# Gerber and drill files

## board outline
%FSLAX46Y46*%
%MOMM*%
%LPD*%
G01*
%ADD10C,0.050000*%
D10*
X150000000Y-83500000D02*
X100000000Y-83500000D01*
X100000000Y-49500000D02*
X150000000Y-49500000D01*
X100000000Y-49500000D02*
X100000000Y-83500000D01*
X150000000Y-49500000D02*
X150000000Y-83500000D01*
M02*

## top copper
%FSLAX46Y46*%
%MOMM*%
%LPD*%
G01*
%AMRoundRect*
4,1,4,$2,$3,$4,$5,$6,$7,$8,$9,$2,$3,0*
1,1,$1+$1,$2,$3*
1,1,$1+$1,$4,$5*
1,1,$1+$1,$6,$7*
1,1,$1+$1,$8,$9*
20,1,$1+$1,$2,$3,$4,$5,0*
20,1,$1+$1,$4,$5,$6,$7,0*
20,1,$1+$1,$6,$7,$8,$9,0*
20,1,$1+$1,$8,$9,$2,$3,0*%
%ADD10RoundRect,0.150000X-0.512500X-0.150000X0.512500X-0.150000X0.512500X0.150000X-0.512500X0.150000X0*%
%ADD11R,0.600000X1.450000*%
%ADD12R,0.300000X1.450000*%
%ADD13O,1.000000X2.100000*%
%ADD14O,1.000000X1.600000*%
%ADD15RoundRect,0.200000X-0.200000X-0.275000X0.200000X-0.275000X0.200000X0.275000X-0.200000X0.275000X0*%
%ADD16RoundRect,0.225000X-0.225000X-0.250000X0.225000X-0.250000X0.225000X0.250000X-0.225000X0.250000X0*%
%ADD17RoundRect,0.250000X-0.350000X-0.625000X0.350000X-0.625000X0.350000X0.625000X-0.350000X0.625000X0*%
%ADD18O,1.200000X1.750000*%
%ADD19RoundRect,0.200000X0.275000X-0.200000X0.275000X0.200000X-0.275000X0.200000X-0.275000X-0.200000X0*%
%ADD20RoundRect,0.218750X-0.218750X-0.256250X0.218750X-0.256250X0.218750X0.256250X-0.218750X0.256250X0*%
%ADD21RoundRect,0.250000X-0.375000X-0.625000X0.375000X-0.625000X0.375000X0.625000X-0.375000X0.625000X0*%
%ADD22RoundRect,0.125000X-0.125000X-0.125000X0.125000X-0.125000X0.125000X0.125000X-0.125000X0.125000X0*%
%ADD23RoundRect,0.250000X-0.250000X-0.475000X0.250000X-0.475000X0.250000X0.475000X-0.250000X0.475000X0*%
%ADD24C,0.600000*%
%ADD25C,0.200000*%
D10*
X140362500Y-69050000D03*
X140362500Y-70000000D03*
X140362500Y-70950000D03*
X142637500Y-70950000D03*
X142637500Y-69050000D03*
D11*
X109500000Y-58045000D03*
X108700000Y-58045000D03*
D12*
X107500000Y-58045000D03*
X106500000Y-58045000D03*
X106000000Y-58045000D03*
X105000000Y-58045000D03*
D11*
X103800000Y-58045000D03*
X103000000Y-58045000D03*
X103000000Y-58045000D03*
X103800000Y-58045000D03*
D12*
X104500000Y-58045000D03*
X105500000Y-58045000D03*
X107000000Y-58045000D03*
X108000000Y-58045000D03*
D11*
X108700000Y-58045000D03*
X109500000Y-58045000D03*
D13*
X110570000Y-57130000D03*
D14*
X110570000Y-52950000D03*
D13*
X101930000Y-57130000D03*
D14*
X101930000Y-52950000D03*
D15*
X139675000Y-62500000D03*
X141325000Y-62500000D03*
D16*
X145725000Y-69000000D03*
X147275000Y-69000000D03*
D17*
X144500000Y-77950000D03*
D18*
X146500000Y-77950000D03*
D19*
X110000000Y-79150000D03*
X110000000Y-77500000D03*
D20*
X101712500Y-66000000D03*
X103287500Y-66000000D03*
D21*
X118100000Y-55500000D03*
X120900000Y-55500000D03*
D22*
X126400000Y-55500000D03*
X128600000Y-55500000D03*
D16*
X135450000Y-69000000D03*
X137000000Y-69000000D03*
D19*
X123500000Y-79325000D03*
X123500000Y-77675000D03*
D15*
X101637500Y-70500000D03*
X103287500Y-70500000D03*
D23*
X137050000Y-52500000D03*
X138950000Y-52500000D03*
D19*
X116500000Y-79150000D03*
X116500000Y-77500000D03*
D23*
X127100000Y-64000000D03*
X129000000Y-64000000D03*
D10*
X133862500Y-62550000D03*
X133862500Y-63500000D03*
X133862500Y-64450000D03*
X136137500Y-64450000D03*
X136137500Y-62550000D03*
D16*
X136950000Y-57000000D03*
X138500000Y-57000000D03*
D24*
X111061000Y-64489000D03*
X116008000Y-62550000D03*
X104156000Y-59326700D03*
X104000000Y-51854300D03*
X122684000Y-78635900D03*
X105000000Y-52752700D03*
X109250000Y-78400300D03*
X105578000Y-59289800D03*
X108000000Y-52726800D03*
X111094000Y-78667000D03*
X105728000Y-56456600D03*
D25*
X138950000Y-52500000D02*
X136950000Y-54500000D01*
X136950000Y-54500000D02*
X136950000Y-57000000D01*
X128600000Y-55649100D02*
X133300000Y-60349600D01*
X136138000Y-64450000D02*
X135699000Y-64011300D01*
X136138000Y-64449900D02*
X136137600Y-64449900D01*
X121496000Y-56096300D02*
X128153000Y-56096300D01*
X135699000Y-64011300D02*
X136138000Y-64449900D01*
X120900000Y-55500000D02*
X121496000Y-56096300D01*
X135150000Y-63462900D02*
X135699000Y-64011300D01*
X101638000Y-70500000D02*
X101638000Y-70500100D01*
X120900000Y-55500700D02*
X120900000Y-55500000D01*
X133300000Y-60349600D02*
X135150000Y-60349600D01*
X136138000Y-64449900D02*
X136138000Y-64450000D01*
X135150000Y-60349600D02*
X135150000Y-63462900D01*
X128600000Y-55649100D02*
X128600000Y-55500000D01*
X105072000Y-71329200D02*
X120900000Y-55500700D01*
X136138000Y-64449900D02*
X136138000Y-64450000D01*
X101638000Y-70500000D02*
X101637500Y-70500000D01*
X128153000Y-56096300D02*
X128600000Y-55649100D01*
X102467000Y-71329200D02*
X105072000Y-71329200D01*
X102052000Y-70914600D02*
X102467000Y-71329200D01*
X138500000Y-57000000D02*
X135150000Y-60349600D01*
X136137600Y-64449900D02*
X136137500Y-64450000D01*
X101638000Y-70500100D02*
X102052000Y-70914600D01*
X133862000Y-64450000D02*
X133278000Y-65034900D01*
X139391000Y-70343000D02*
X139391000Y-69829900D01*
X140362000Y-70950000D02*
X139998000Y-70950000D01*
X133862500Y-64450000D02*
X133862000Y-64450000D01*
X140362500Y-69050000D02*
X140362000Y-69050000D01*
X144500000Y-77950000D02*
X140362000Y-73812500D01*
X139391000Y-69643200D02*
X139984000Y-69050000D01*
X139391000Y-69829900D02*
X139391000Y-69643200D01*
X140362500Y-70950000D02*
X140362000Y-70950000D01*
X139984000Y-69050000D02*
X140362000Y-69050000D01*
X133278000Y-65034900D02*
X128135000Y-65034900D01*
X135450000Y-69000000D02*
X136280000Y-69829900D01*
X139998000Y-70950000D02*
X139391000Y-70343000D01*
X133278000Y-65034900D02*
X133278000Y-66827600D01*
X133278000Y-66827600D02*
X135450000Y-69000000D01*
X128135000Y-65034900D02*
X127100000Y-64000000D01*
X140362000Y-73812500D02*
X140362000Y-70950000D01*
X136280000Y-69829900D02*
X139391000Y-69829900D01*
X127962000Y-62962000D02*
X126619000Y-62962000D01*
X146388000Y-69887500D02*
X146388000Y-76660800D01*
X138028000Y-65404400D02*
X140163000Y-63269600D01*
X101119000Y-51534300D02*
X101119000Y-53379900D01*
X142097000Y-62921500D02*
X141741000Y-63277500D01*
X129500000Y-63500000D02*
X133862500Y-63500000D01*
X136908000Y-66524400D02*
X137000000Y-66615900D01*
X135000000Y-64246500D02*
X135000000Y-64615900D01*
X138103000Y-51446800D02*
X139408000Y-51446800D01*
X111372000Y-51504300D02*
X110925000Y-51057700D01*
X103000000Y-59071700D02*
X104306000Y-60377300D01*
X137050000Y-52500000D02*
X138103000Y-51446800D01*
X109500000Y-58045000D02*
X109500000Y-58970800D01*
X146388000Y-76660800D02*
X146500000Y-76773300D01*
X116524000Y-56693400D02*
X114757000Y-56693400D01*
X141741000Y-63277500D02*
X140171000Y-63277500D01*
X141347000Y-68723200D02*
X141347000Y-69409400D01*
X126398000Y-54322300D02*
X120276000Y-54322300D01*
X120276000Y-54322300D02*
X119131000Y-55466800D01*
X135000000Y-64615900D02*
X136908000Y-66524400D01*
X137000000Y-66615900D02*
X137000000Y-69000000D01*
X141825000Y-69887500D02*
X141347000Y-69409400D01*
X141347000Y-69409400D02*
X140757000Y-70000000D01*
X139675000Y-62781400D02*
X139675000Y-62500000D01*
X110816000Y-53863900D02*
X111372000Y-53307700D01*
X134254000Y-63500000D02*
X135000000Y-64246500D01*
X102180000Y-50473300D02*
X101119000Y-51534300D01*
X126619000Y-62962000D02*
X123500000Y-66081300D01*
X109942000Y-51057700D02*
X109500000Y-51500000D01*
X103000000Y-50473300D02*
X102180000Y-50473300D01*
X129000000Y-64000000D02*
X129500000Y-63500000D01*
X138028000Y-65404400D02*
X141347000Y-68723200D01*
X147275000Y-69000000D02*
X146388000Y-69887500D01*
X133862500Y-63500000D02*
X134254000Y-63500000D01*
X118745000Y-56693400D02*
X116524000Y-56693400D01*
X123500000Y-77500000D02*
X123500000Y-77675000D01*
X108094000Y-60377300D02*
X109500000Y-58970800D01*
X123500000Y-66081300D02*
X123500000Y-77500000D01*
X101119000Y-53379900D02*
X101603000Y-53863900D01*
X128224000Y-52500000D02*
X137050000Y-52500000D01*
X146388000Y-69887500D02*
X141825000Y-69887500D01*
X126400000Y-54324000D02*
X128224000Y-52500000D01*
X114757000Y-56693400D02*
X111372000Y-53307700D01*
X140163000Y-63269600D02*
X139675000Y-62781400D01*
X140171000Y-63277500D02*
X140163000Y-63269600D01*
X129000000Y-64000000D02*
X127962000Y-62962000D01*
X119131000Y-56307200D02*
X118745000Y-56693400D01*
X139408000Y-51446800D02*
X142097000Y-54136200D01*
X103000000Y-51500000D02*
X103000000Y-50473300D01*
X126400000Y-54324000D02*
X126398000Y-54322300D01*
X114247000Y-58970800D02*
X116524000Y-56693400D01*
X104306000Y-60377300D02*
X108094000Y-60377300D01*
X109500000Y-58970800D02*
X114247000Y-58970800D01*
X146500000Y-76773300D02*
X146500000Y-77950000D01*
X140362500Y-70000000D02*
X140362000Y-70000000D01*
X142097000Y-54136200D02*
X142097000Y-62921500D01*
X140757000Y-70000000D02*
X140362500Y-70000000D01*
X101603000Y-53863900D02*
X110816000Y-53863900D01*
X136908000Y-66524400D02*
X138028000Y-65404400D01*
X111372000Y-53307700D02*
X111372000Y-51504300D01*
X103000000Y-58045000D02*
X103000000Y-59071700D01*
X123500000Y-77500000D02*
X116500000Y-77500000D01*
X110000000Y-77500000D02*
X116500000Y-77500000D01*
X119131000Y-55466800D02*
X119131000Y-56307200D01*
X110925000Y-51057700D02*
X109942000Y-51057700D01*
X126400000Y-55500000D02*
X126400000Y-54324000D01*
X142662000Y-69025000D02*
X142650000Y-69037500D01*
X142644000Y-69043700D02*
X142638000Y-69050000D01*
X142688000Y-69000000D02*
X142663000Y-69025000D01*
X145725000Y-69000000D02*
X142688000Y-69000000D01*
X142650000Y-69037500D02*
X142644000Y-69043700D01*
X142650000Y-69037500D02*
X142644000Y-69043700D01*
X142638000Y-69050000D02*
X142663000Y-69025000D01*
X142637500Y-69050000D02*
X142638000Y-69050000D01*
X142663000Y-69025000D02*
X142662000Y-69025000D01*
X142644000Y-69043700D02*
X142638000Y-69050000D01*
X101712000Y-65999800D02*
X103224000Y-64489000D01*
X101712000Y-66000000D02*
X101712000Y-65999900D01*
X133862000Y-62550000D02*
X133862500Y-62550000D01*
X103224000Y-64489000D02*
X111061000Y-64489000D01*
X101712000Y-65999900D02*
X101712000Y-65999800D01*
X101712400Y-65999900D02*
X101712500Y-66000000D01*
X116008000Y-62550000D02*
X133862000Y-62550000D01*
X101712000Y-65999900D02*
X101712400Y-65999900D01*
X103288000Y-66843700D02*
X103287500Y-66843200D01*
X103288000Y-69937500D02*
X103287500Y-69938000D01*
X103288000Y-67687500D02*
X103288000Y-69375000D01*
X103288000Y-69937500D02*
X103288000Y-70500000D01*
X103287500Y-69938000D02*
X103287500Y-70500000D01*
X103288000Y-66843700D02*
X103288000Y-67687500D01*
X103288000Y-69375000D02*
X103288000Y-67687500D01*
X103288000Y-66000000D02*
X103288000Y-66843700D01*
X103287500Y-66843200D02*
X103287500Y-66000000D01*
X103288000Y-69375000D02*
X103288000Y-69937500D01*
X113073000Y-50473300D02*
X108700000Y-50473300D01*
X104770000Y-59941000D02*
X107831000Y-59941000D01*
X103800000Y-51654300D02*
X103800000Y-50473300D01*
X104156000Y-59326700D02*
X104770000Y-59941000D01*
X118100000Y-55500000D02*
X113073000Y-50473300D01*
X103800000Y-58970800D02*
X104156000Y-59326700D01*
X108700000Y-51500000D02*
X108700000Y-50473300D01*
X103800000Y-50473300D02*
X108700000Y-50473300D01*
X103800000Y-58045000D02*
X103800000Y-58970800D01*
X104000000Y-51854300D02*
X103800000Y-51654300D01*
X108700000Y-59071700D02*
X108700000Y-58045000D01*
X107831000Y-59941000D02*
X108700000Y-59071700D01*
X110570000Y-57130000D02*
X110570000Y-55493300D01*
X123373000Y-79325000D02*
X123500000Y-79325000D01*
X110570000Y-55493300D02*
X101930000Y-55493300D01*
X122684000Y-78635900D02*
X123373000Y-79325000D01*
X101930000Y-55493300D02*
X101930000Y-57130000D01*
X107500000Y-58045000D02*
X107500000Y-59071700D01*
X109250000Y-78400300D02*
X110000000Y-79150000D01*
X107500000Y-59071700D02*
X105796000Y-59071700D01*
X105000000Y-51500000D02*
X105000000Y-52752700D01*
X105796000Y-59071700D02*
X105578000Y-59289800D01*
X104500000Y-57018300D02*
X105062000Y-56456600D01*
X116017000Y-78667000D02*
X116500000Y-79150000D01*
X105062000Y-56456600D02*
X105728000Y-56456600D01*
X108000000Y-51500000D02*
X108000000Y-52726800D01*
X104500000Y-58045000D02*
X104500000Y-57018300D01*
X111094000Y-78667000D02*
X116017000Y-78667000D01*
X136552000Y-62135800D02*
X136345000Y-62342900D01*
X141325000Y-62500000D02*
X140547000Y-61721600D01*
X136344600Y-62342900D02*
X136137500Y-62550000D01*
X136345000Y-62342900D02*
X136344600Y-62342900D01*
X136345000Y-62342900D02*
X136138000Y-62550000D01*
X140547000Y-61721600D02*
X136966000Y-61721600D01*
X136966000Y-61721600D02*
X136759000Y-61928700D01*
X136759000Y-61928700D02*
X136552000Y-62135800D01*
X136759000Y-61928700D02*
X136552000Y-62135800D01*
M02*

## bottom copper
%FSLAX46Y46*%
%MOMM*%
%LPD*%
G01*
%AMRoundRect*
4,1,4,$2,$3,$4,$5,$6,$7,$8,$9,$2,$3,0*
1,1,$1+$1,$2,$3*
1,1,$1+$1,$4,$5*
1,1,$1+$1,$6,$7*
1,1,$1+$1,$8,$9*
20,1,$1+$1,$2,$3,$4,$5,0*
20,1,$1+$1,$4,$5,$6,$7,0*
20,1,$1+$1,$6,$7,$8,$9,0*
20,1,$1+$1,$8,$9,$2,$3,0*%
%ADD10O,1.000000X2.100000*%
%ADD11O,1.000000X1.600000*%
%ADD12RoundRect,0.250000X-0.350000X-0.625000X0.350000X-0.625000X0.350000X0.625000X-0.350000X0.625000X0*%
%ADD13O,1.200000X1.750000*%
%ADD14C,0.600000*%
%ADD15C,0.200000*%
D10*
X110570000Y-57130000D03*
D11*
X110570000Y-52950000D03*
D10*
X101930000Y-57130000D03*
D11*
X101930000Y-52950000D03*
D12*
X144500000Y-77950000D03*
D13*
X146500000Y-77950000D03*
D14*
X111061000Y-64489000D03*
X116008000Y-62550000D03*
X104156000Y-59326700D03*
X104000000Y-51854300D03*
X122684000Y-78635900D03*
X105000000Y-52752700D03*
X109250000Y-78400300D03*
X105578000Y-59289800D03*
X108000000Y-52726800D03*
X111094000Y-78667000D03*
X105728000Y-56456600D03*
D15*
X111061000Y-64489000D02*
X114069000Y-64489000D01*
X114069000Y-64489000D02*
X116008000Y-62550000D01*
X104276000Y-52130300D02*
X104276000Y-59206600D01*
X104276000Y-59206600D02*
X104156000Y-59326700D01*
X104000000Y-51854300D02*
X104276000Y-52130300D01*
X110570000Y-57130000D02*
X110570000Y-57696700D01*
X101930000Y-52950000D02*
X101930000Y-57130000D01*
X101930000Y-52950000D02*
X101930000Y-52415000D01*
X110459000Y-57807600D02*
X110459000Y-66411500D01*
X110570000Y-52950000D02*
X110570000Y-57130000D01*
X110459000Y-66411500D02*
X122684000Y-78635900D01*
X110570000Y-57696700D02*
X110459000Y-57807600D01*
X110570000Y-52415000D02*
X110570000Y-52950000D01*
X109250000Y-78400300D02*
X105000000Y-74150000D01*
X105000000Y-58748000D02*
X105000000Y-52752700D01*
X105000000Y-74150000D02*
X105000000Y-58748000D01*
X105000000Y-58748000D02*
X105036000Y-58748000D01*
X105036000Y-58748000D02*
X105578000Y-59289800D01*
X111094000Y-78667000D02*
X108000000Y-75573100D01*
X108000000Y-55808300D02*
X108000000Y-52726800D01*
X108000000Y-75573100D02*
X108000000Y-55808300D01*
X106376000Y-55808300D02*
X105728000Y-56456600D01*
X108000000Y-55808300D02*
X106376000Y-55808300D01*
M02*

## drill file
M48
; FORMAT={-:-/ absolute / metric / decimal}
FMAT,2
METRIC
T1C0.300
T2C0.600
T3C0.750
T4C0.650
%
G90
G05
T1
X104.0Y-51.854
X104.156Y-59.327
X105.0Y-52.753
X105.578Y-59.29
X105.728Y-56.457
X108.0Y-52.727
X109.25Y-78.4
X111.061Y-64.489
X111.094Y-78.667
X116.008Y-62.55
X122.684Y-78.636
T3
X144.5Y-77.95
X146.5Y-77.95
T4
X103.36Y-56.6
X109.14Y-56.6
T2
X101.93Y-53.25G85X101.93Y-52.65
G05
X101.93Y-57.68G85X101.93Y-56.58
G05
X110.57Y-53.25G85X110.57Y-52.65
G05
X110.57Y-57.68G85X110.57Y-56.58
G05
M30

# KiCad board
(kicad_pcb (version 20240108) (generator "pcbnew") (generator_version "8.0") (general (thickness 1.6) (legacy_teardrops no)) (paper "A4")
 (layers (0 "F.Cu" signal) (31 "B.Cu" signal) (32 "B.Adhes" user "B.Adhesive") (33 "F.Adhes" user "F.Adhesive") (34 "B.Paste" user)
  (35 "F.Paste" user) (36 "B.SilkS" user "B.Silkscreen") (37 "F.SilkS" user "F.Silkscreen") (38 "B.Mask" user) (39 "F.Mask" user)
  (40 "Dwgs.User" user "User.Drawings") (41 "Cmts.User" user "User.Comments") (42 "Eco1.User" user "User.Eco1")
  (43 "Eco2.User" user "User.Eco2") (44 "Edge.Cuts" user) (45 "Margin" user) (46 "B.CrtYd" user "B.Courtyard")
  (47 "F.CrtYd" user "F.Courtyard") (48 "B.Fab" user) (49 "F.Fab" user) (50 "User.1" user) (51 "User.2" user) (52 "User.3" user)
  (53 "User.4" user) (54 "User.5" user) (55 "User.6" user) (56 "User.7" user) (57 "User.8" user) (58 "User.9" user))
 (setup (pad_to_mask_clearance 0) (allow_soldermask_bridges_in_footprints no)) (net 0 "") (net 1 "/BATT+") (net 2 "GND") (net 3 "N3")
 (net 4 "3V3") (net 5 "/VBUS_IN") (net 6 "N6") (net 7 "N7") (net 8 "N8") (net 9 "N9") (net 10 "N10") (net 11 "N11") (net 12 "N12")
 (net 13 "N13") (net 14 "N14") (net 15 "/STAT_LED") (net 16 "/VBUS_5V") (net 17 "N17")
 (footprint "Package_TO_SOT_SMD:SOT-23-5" (layer "F.Cu") (at 141.5 70)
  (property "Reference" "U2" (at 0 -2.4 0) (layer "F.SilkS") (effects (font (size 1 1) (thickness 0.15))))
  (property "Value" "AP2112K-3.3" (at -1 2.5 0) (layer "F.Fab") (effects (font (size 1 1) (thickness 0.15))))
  (pad "1" smd roundrect (at -1.1375 -0.95) (size 1.325 0.6) (layers "F.Cu" "F.Paste" "F.Mask") (roundrect_rratio 0.25) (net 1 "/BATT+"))
  (pad "2" smd roundrect (at -1.1375 0) (size 1.325 0.6) (layers "F.Cu" "F.Paste" "F.Mask") (roundrect_rratio 0.25) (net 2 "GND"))
  (pad "3" smd roundrect (at -1.1375 0.95) (size 1.325 0.6) (layers "F.Cu" "F.Paste" "F.Mask") (roundrect_rratio 0.25) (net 1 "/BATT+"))
  (pad "4" smd roundrect (at 1.1375 0.95) (size 1.325 0.6) (layers "F.Cu" "F.Paste" "F.Mask") (roundrect_rratio 0.25) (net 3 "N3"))
  (pad "5" smd roundrect (at 1.1375 -0.95) (size 1.325 0.6) (layers "F.Cu" "F.Paste" "F.Mask") (roundrect_rratio 0.25) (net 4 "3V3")))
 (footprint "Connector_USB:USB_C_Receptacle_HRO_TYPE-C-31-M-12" (layer "F.Cu") (at 106.25 54 180)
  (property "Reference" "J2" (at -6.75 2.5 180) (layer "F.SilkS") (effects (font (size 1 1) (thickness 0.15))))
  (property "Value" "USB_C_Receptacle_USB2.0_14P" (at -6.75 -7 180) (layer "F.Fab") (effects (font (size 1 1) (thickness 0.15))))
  (pad "" np_thru_hole circle (at -2.89 -2.6 180) (size 0.65 0.65) (drill 0.65) (layers "*.Cu" "*.Mask"))
  (pad "" np_thru_hole circle (at 2.89 -2.6 180) (size 0.65 0.65) (drill 0.65) (layers "*.Cu" "*.Mask"))
  (pad "A1" smd rect (at -3.25 -4.045 180) (size 0.6 1.45) (layers "F.Cu" "F.Paste" "F.Mask") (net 2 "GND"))
  (pad "A4" smd rect (at -2.45 -4.045 180) (size 0.6 1.45) (layers "F.Cu" "F.Paste" "F.Mask") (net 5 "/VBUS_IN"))
  (pad "A5" smd rect (at -1.25 -4.045 180) (size 0.3 1.45) (layers "F.Cu" "F.Paste" "F.Mask") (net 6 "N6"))
  (pad "A6" smd rect (at -0.25 -4.045 180) (size 0.3 1.45) (layers "F.Cu" "F.Paste" "F.Mask") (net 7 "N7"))
  (pad "A7" smd rect (at 0.25 -4.045 180) (size 0.3 1.45) (layers "F.Cu" "F.Paste" "F.Mask") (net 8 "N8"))
  (pad "A8" smd rect (at 1.25 -4.045 180) (size 0.3 1.45) (layers "F.Cu" "F.Paste" "F.Mask"))
  (pad "A9" smd rect (at 2.45 -4.045 180) (size 0.6 1.45) (layers "F.Cu" "F.Paste" "F.Mask") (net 5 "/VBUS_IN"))
  (pad "A12" smd rect (at 3.25 -4.045 180) (size 0.6 1.45) (layers "F.Cu" "F.Paste" "F.Mask") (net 2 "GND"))
  (pad "B1" smd rect (at 3.25 -4.045 180) (size 0.6 1.45) (layers "F.Cu" "F.Paste" "F.Mask") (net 2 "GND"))
  (pad "B4" smd rect (at 2.45 -4.045 180) (size 0.6 1.45) (layers "F.Cu" "F.Paste" "F.Mask") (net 5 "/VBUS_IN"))
  (pad "B5" smd rect (at 1.75 -4.045 180) (size 0.3 1.45) (layers "F.Cu" "F.Paste" "F.Mask") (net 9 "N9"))
  (pad "B6" smd rect (at 0.75 -4.045 180) (size 0.3 1.45) (layers "F.Cu" "F.Paste" "F.Mask") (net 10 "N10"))
  (pad "B7" smd rect (at -0.75 -4.045 180) (size 0.3 1.45) (layers "F.Cu" "F.Paste" "F.Mask") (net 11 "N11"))
  (pad "B8" smd rect (at -1.75 -4.045 180) (size 0.3 1.45) (layers "F.Cu" "F.Paste" "F.Mask"))
  (pad "B9" smd rect (at -2.45 -4.045 180) (size 0.6 1.45) (layers "F.Cu" "F.Paste" "F.Mask") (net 5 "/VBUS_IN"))
  (pad "B12" smd rect (at -3.25 -4.045 180) (size 0.6 1.45) (layers "F.Cu" "F.Paste" "F.Mask") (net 2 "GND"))
  (pad "S1" thru_hole oval (at -4.32 -3.13 180) (size 1 2.1) (drill oval 0.6 1.7) (layers "*.Cu" "*.Mask") (remove_unused_layers no)
   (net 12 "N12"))
  (pad "S1" thru_hole oval (at -4.32 1.05 180) (size 1 1.6) (drill oval 0.6 1.2) (layers "*.Cu" "*.Mask") (remove_unused_layers no)
   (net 12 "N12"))
  (pad "S1" thru_hole oval (at 4.32 -3.13 180) (size 1 2.1) (drill oval 0.6 1.7) (layers "*.Cu" "*.Mask") (remove_unused_layers no)
   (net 12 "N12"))
  (pad "S1" thru_hole oval (at 4.32 1.05 180) (size 1 1.6) (drill oval 0.6 1.2) (layers "*.Cu" "*.Mask") (remove_unused_layers no)
   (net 12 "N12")))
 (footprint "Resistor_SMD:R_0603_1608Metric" (layer "F.Cu") (at 140.5 62.5)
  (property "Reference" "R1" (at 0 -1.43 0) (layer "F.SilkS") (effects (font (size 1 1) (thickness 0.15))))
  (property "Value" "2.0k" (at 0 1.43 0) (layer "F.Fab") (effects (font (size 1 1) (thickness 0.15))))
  (pad "1" smd roundrect (at -0.825 0) (size 0.8 0.95) (layers "F.Cu" "F.Paste" "F.Mask") (roundrect_rratio 0.25) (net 2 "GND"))
  (pad "2" smd roundrect (at 0.825 0) (size 0.8 0.95) (layers "F.Cu" "F.Paste" "F.Mask") (roundrect_rratio 0.25) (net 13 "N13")))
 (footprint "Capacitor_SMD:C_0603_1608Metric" (layer "F.Cu") (at 146.5 69)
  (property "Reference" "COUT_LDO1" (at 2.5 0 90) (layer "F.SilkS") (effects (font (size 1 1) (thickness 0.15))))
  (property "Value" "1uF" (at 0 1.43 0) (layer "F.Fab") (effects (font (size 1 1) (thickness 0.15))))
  (pad "1" smd roundrect (at -0.775 0) (size 0.9 0.95) (layers "F.Cu" "F.Paste" "F.Mask") (roundrect_rratio 0.25) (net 4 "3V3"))
  (pad "2" smd roundrect (at 0.775 0) (size 0.9 0.95) (layers "F.Cu" "F.Paste" "F.Mask") (roundrect_rratio 0.25) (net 2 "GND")))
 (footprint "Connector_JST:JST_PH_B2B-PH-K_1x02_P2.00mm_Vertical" (layer "F.Cu") (at 144.5 77.95)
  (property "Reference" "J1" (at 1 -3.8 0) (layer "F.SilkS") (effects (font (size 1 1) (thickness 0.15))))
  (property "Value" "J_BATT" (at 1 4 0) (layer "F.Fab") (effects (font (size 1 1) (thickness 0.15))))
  (pad "1" thru_hole roundrect (at 0 0) (size 1.2 1.75) (drill 0.75) (layers "*.Cu" "*.Mask") (remove_unused_layers no)
   (roundrect_rratio 0.208333) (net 1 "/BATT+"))
  (pad "2" thru_hole oval (at 2 0) (size 1.2 1.75) (drill 0.75) (layers "*.Cu" "*.Mask") (remove_unused_layers no) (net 2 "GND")))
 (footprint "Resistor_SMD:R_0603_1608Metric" (layer "F.Cu") (at 110 78.325 90)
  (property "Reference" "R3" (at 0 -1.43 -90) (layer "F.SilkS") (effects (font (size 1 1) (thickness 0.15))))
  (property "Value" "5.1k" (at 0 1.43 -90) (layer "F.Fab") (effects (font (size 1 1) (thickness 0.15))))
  (pad "1" smd roundrect (at -0.825 0 90) (size 0.8 0.95) (layers "F.Cu" "F.Paste" "F.Mask") (roundrect_rratio 0.25) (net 6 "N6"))
  (pad "2" smd roundrect (at 0.825 0 90) (size 0.8 0.95) (layers "F.Cu" "F.Paste" "F.Mask") (roundrect_rratio 0.25) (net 2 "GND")))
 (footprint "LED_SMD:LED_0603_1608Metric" (layer "F.Cu") (at 102.5 66)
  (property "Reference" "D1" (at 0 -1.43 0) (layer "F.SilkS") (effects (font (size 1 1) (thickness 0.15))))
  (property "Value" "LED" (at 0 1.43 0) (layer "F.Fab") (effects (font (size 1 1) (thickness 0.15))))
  (pad "1" smd roundrect (at -0.7875 0) (size 0.875 0.95) (layers "F.Cu" "F.Paste" "F.Mask") (roundrect_rratio 0.25) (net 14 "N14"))
  (pad "2" smd roundrect (at 0.7875 0) (size 0.875 0.95) (layers "F.Cu" "F.Paste" "F.Mask") (roundrect_rratio 0.25) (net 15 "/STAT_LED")))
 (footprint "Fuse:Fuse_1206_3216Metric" (layer "F.Cu") (at 119.5 55.5)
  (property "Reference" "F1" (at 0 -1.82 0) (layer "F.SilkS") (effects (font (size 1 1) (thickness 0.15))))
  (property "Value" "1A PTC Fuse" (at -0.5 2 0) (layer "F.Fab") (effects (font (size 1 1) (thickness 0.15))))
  (pad "1" smd roundrect (at -1.4 0) (size 1.25 1.75) (layers "F.Cu" "F.Paste" "F.Mask") (roundrect_rratio 0.2) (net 5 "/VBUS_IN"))
  (pad "2" smd roundrect (at 1.4 0) (size 1.25 1.75) (layers "F.Cu" "F.Paste" "F.Mask") (roundrect_rratio 0.2) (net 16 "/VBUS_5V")))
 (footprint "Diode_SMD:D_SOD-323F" (layer "F.Cu") (at 127.5 55.5)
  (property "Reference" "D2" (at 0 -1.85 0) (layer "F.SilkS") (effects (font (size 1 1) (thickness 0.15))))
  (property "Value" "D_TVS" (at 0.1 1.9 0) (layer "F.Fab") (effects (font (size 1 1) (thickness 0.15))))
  (pad "1" smd roundrect (at -1.1 0) (size 0.5 0.5) (layers "F.Cu" "F.Paste" "F.Mask") (roundrect_rratio 0.25) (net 2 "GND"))
  (pad "2" smd roundrect (at 1.1 0) (size 0.5 0.5) (layers "F.Cu" "F.Paste" "F.Mask") (roundrect_rratio 0.25) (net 16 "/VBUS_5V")))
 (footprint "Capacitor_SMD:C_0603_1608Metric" (layer "F.Cu") (at 136.225 69)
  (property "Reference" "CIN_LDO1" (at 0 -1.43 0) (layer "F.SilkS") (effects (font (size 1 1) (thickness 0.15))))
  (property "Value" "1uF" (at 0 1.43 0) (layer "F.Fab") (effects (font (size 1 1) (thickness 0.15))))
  (pad "1" smd roundrect (at -0.775 0) (size 0.9 0.95) (layers "F.Cu" "F.Paste" "F.Mask") (roundrect_rratio 0.25) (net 1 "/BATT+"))
  (pad "2" smd roundrect (at 0.775 0) (size 0.9 0.95) (layers "F.Cu" "F.Paste" "F.Mask") (roundrect_rratio 0.25) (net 2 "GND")))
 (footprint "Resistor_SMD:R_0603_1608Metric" (layer "F.Cu") (at 123.5 78.5 90)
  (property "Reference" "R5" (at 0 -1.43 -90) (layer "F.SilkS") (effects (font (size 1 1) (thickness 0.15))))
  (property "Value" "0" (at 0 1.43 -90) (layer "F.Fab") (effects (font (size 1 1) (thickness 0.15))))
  (pad "1" smd roundrect (at -0.825 0 90) (size 0.8 0.95) (layers "F.Cu" "F.Paste" "F.Mask") (roundrect_rratio 0.25) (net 12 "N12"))
  (pad "2" smd roundrect (at 0.825 0 90) (size 0.8 0.95) (layers "F.Cu" "F.Paste" "F.Mask") (roundrect_rratio 0.25) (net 2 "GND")))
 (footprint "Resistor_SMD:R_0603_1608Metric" (layer "F.Cu") (at 102.4625 70.5)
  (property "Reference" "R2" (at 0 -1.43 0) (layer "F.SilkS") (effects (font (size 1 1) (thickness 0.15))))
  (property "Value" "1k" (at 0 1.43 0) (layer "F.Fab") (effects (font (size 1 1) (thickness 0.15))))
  (pad "1" smd roundrect (at -0.825 0) (size 0.8 0.95) (layers "F.Cu" "F.Paste" "F.Mask") (roundrect_rratio 0.25) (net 16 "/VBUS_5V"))
  (pad "2" smd roundrect (at 0.825 0) (size 0.8 0.95) (layers "F.Cu" "F.Paste" "F.Mask") (roundrect_rratio 0.25) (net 15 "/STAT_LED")))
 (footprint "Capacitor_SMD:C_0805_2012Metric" (layer "F.Cu") (at 138 52.5)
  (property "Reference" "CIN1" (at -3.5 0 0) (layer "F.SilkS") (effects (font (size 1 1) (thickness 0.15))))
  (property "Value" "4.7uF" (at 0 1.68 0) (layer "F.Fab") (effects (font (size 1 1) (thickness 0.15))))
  (pad "1" smd roundrect (at -0.95 0) (size 1 1.45) (layers "F.Cu" "F.Paste" "F.Mask") (roundrect_rratio 0.25) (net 2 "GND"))
  (pad "2" smd roundrect (at 0.95 0) (size 1 1.45) (layers "F.Cu" "F.Paste" "F.Mask") (roundrect_rratio 0.25) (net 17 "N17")))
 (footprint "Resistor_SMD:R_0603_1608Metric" (layer "F.Cu") (at 116.5 78.325 90)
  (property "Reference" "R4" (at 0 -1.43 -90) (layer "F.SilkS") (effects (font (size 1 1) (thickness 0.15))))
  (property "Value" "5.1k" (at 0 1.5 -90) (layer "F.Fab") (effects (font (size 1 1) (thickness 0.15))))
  (pad "1" smd roundrect (at -0.825 0 90) (size 0.8 0.95) (layers "F.Cu" "F.Paste" "F.Mask") (roundrect_rratio 0.25) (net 9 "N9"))
  (pad "2" smd roundrect (at 0.825 0 90) (size 0.8 0.95) (layers "F.Cu" "F.Paste" "F.Mask") (roundrect_rratio 0.25) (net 2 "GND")))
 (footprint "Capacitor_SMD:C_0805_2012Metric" (layer "F.Cu") (at 128.05 64)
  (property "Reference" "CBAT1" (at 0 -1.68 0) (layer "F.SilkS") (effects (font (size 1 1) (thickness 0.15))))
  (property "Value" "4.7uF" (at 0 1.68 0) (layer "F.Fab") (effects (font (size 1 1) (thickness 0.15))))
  (pad "1" smd roundrect (at -0.95 0) (size 1 1.45) (layers "F.Cu" "F.Paste" "F.Mask") (roundrect_rratio 0.25) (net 1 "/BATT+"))
  (pad "2" smd roundrect (at 0.95 0) (size 1 1.45) (layers "F.Cu" "F.Paste" "F.Mask") (roundrect_rratio 0.25) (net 2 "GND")))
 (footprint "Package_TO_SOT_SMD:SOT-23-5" (layer "F.Cu") (at 135 63.5)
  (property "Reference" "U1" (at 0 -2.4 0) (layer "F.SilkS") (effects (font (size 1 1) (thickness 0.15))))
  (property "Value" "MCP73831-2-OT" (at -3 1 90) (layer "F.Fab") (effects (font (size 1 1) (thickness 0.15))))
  (pad "1" smd roundrect (at -1.1375 -0.95) (size 1.325 0.6) (layers "F.Cu" "F.Paste" "F.Mask") (roundrect_rratio 0.25) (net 14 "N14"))
  (pad "2" smd roundrect (at -1.1375 0) (size 1.325 0.6) (layers "F.Cu" "F.Paste" "F.Mask") (roundrect_rratio 0.25) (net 2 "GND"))
  (pad "3" smd roundrect (at -1.1375 0.95) (size 1.325 0.6) (layers "F.Cu" "F.Paste" "F.Mask") (roundrect_rratio 0.25) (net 1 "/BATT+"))
  (pad "4" smd roundrect (at 1.1375 0.95) (size 1.325 0.6) (layers "F.Cu" "F.Paste" "F.Mask") (roundrect_rratio 0.25) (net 16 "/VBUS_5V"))
  (pad "5" smd roundrect (at 1.1375 -0.95) (size 1.325 0.6) (layers "F.Cu" "F.Paste" "F.Mask") (roundrect_rratio 0.25) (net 13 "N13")))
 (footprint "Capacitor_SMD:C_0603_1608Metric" (layer "F.Cu") (at 137.725 57)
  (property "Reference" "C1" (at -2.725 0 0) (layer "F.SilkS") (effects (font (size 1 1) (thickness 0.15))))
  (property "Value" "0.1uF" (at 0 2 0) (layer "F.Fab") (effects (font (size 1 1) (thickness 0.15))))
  (pad "1" smd roundrect (at -0.775 0) (size 0.9 0.95) (layers "F.Cu" "F.Paste" "F.Mask") (roundrect_rratio 0.25) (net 17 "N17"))
  (pad "2" smd roundrect (at 0.775 0) (size 0.9 0.95) (layers "F.Cu" "F.Paste" "F.Mask") (roundrect_rratio 0.25) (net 16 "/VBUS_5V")))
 (gr_line (start 150 83.5) (end 100 83.5) (stroke (width 0.05) (type default)) (layer "Edge.Cuts"))
 (gr_line (start 100 49.5) (end 150 49.5) (stroke (width 0.05) (type default)) (layer "Edge.Cuts"))
 (gr_line (start 100 49.5) (end 100 83.5) (stroke (width 0.05) (type default)) (layer "Edge.Cuts"))
 (gr_line (start 150 49.5) (end 150 83.5) (stroke (width 0.05) (type default)) (layer "Edge.Cuts"))
 (segment (start 138.95 52.5) (end 136.95 54.5) (width 0.2) (layer "F.Cu") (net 17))
 (segment (start 136.95 54.5) (end 136.95 57) (width 0.2) (layer "F.Cu") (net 17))
 (segment (start 128.6 55.6491) (end 133.3 60.3496) (width 0.2) (layer "F.Cu") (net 16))
 (segment (start 136.138 64.45) (end 135.699 64.0113) (width 0.2) (layer "F.Cu") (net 16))
 (segment (start 136.138 64.4499) (end 136.1376 64.4499) (width 0.2) (layer "F.Cu") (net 16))
 (segment (start 121.496 56.0963) (end 128.153 56.0963) (width 0.2) (layer "F.Cu") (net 16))
 (segment (start 135.699 64.0113) (end 136.138 64.4499) (width 0.2) (layer "F.Cu") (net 16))
 (segment (start 120.9 55.5) (end 121.496 56.0963) (width 0.2) (layer "F.Cu") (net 16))
 (segment (start 135.15 63.4629) (end 135.699 64.0113) (width 0.2) (layer "F.Cu") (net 16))
 (segment (start 101.638 70.5) (end 101.638 70.5001) (width 0.2) (layer "F.Cu") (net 16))
 (segment (start 120.9 55.5007) (end 120.9 55.5) (width 0.2) (layer "F.Cu") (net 16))
 (segment (start 133.3 60.3496) (end 135.15 60.3496) (width 0.2) (layer "F.Cu") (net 16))
 (segment (start 136.138 64.4499) (end 136.138 64.45) (width 0.2) (layer "F.Cu") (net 16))
 (segment (start 135.15 60.3496) (end 135.15 63.4629) (width 0.2) (layer "F.Cu") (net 16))
 (segment (start 128.6 55.6491) (end 128.6 55.5) (width 0.2) (layer "F.Cu") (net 16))
 (segment (start 105.072 71.3292) (end 120.9 55.5007) (width 0.2) (layer "F.Cu") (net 16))
 (segment (start 136.138 64.4499) (end 136.138 64.45) (width 0.2) (layer "F.Cu") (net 16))
 (segment (start 101.638 70.5) (end 101.6375 70.5) (width 0.2) (layer "F.Cu") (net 16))
 (segment (start 128.153 56.0963) (end 128.6 55.6491) (width 0.2) (layer "F.Cu") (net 16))
 (segment (start 102.467 71.3292) (end 105.072 71.3292) (width 0.2) (layer "F.Cu") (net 16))
 (segment (start 102.052 70.9146) (end 102.467 71.3292) (width 0.2) (layer "F.Cu") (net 16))
 (segment (start 138.5 57) (end 135.15 60.3496) (width 0.2) (layer "F.Cu") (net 16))
 (segment (start 136.1376 64.4499) (end 136.1375 64.45) (width 0.2) (layer "F.Cu") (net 16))
 (segment (start 101.638 70.5001) (end 102.052 70.9146) (width 0.2) (layer "F.Cu") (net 16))
 (segment (start 133.862 64.45) (end 133.278 65.0349) (width 0.2) (layer "F.Cu") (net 1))
 (segment (start 139.391 70.343) (end 139.391 69.8299) (width 0.2) (layer "F.Cu") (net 1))
 (segment (start 140.362 70.95) (end 139.998 70.95) (width 0.2) (layer "F.Cu") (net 1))
 (segment (start 133.8625 64.45) (end 133.862 64.45) (width 0.2) (layer "F.Cu") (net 1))
 (segment (start 140.3625 69.05) (end 140.362 69.05) (width 0.2) (layer "F.Cu") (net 1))
 (segment (start 144.5 77.95) (end 140.362 73.8125) (width 0.2) (layer "F.Cu") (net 1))
 (segment (start 139.391 69.6432) (end 139.984 69.05) (width 0.2) (layer "F.Cu") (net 1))
 (segment (start 139.391 69.8299) (end 139.391 69.6432) (width 0.2) (layer "F.Cu") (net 1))
 (segment (start 140.3625 70.95) (end 140.362 70.95) (width 0.2) (layer "F.Cu") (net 1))
 (segment (start 139.984 69.05) (end 140.362 69.05) (width 0.2) (layer "F.Cu") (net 1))
 (segment (start 133.278 65.0349) (end 128.135 65.0349) (width 0.2) (layer "F.Cu") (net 1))
 (segment (start 135.45 69) (end 136.28 69.8299) (width 0.2) (layer "F.Cu") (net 1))
 (segment (start 139.998 70.95) (end 139.391 70.343) (width 0.2) (layer "F.Cu") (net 1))
 (segment (start 133.278 65.0349) (end 133.278 66.8276) (width 0.2) (layer "F.Cu") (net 1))
 (segment (start 133.278 66.8276) (end 135.45 69) (width 0.2) (layer "F.Cu") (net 1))
 (segment (start 128.135 65.0349) (end 127.1 64) (width 0.2) (layer "F.Cu") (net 1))
 (segment (start 140.362 73.8125) (end 140.362 70.95) (width 0.2) (layer "F.Cu") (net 1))
 (segment (start 136.28 69.8299) (end 139.391 69.8299) (width 0.2) (layer "F.Cu") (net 1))
 (segment (start 127.962 62.962) (end 126.619 62.962) (width 0.2) (layer "F.Cu") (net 2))
 (segment (start 146.388 69.8875) (end 146.388 76.6608) (width 0.2) (layer "F.Cu") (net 2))
 (segment (start 138.028 65.4044) (end 140.163 63.2696) (width 0.2) (layer "F.Cu") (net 2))
 (segment (start 101.119 51.5343) (end 101.119 53.3799) (width 0.2) (layer "F.Cu") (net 2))
 (segment (start 142.097 62.9215) (end 141.741 63.2775) (width 0.2) (layer "F.Cu") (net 2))
 (segment (start 129.5 63.5) (end 133.8625 63.5) (width 0.2) (layer "F.Cu") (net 2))
 (segment (start 136.908 66.5244) (end 137 66.6159) (width 0.2) (layer "F.Cu") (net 2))
 (segment (start 135 64.2465) (end 135 64.6159) (width 0.2) (layer "F.Cu") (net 2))
 (segment (start 138.103 51.4468) (end 139.408 51.4468) (width 0.2) (layer "F.Cu") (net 2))
 (segment (start 111.372 51.5043) (end 110.925 51.0577) (width 0.2) (layer "F.Cu") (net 2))
 (segment (start 103 59.0717) (end 104.306 60.3773) (width 0.2) (layer "F.Cu") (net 2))
 (segment (start 137.05 52.5) (end 138.103 51.4468) (width 0.2) (layer "F.Cu") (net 2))
 (segment (start 109.5 58.045) (end 109.5 58.9708) (width 0.2) (layer "F.Cu") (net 2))
 (segment (start 146.388 76.6608) (end 146.5 76.7733) (width 0.2) (layer "F.Cu") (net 2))
 (segment (start 116.524 56.6934) (end 114.757 56.6934) (width 0.2) (layer "F.Cu") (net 2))
 (segment (start 141.741 63.2775) (end 140.171 63.2775) (width 0.2) (layer "F.Cu") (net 2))
 (segment (start 141.347 68.7232) (end 141.347 69.4094) (width 0.2) (layer "F.Cu") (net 2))
 (segment (start 126.398 54.3223) (end 120.276 54.3223) (width 0.2) (layer "F.Cu") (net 2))
 (segment (start 120.276 54.3223) (end 119.131 55.4668) (width 0.2) (layer "F.Cu") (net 2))
 (segment (start 135 64.6159) (end 136.908 66.5244) (width 0.2) (layer "F.Cu") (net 2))
 (segment (start 137 66.6159) (end 137 69) (width 0.2) (layer "F.Cu") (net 2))
 (segment (start 141.825 69.8875) (end 141.347 69.4094) (width 0.2) (layer "F.Cu") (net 2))
 (segment (start 141.347 69.4094) (end 140.757 70) (width 0.2) (layer "F.Cu") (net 2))
 (segment (start 139.675 62.7814) (end 139.675 62.5) (width 0.2) (layer "F.Cu") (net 2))
 (segment (start 110.816 53.8639) (end 111.372 53.3077) (width 0.2) (layer "F.Cu") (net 2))
 (segment (start 134.254 63.5) (end 135 64.2465) (width 0.2) (layer "F.Cu") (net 2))
 (segment (start 102.18 50.4733) (end 101.119 51.5343) (width 0.2) (layer "F.Cu") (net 2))
 (segment (start 126.619 62.962) (end 123.5 66.0813) (width 0.2) (layer "F.Cu") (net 2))
 (segment (start 109.942 51.0577) (end 109.5 51.5) (width 0.2) (layer "F.Cu") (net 2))
 (segment (start 103 50.4733) (end 102.18 50.4733) (width 0.2) (layer "F.Cu") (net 2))
 (segment (start 129 64) (end 129.5 63.5) (width 0.2) (layer "F.Cu") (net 2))
 (segment (start 138.028 65.4044) (end 141.347 68.7232) (width 0.2) (layer "F.Cu") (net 2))
 (segment (start 147.275 69) (end 146.388 69.8875) (width 0.2) (layer "F.Cu") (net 2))
 (segment (start 133.8625 63.5) (end 134.254 63.5) (width 0.2) (layer "F.Cu") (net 2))
 (segment (start 118.745 56.6934) (end 116.524 56.6934) (width 0.2) (layer "F.Cu") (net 2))
 (segment (start 123.5 77.5) (end 123.5 77.675) (width 0.2) (layer "F.Cu") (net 2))
 (segment (start 108.094 60.3773) (end 109.5 58.9708) (width 0.2) (layer "F.Cu") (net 2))
 (segment (start 123.5 66.0813) (end 123.5 77.5) (width 0.2) (layer "F.Cu") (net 2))
 (segment (start 101.119 53.3799) (end 101.603 53.8639) (width 0.2) (layer "F.Cu") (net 2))
 (segment (start 128.224 52.5) (end 137.05 52.5) (width 0.2) (layer "F.Cu") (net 2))
 (segment (start 146.388 69.8875) (end 141.825 69.8875) (width 0.2) (layer "F.Cu") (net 2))
 (segment (start 126.4 54.324) (end 128.224 52.5) (width 0.2) (layer "F.Cu") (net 2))
 (segment (start 114.757 56.6934) (end 111.372 53.3077) (width 0.2) (layer "F.Cu") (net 2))
 (segment (start 140.163 63.2696) (end 139.675 62.7814) (width 0.2) (layer "F.Cu") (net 2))
 (segment (start 140.171 63.2775) (end 140.163 63.2696) (width 0.2) (layer "F.Cu") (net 2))
 (segment (start 129 64) (end 127.962 62.962) (width 0.2) (layer "F.Cu") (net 2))
 (segment (start 119.131 56.3072) (end 118.745 56.6934) (width 0.2) (layer "F.Cu") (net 2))
 (segment (start 139.408 51.4468) (end 142.097 54.1362) (width 0.2) (layer "F.Cu") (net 2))
 (segment (start 103 51.5) (end 103 50.4733) (width 0.2) (layer "F.Cu") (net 2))
 (segment (start 126.4 54.324) (end 126.398 54.3223) (width 0.2) (layer "F.Cu") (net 2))
 (segment (start 114.247 58.9708) (end 116.524 56.6934) (width 0.2) (layer "F.Cu") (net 2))
 (segment (start 104.306 60.3773) (end 108.094 60.3773) (width 0.2) (layer "F.Cu") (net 2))
 (segment (start 109.5 58.9708) (end 114.247 58.9708) (width 0.2) (layer "F.Cu") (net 2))
 (segment (start 146.5 76.7733) (end 146.5 77.95) (width 0.2) (layer "F.Cu") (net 2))
 (segment (start 140.3625 70) (end 140.362 70) (width 0.2) (layer "F.Cu") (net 2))
 (segment (start 142.097 54.1362) (end 142.097 62.9215) (width 0.2) (layer "F.Cu") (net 2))
 (segment (start 140.757 70) (end 140.3625 70) (width 0.2) (layer "F.Cu") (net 2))
 (segment (start 101.603 53.8639) (end 110.816 53.8639) (width 0.2) (layer "F.Cu") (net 2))
 (segment (start 136.908 66.5244) (end 138.028 65.4044) (width 0.2) (layer "F.Cu") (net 2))
 (segment (start 111.372 53.3077) (end 111.372 51.5043) (width 0.2) (layer "F.Cu") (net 2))
 (segment (start 103 58.045) (end 103 59.0717) (width 0.2) (layer "F.Cu") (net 2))
 (segment (start 123.5 77.5) (end 116.5 77.5) (width 0.2) (layer "F.Cu") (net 2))
 (segment (start 110 77.5) (end 116.5 77.5) (width 0.2) (layer "F.Cu") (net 2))
 (segment (start 119.131 55.4668) (end 119.131 56.3072) (width 0.2) (layer "F.Cu") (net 2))
 (segment (start 110.925 51.0577) (end 109.942 51.0577) (width 0.2) (layer "F.Cu") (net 2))
 (segment (start 126.4 55.5) (end 126.4 54.324) (width 0.2) (layer "F.Cu") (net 2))
 (segment (start 142.662 69.025) (end 142.65 69.0375) (width 0.2) (layer "F.Cu") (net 4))
 (segment (start 142.644 69.0437) (end 142.638 69.05) (width 0.2) (layer "F.Cu") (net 4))
 (segment (start 142.688 69) (end 142.663 69.025) (width 0.2) (layer "F.Cu") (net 4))
 (segment (start 145.725 69) (end 142.688 69) (width 0.2) (layer "F.Cu") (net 4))
 (segment (start 142.65 69.0375) (end 142.644 69.0437) (width 0.2) (layer "F.Cu") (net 4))
 (segment (start 142.65 69.0375) (end 142.644 69.0437) (width 0.2) (layer "F.Cu") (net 4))
 (segment (start 142.638 69.05) (end 142.663 69.025) (width 0.2) (layer "F.Cu") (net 4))
 (segment (start 142.6375 69.05) (end 142.638 69.05) (width 0.2) (layer "F.Cu") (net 4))
 (segment (start 142.663 69.025) (end 142.662 69.025) (width 0.2) (layer "F.Cu") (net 4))
 (segment (start 142.644 69.0437) (end 142.638 69.05) (width 0.2) (layer "F.Cu") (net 4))
 (segment (start 101.712 65.9998) (end 103.224 64.489) (width 0.2) (layer "F.Cu") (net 14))
 (segment (start 101.712 66) (end 101.712 65.9999) (width 0.2) (layer "F.Cu") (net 14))
 (segment (start 133.862 62.55) (end 133.8625 62.55) (width 0.2) (layer "F.Cu") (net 14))
 (segment (start 103.224 64.489) (end 111.061 64.489) (width 0.2) (layer "F.Cu") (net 14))
 (segment (start 101.712 65.9999) (end 101.712 65.9998) (width 0.2) (layer "F.Cu") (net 14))
 (segment (start 101.7124 65.9999) (end 101.7125 66) (width 0.2) (layer "F.Cu") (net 14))
 (segment (start 116.008 62.55) (end 133.862 62.55) (width 0.2) (layer "F.Cu") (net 14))
 (segment (start 101.712 65.9999) (end 101.7124 65.9999) (width 0.2) (layer "F.Cu") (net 14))
 (via (at 111.061 64.489) (size 0.6) (drill 0.3) (layers "F.Cu" "B.Cu") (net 14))
 (via (at 116.008 62.55) (size 0.6) (drill 0.3) (layers "F.Cu" "B.Cu") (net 14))
 (segment (start 111.061 64.489) (end 114.069 64.489) (width 0.2) (layer "B.Cu") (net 14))
 (segment (start 114.069 64.489) (end 116.008 62.55) (width 0.2) (layer "B.Cu") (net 14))
 (segment (start 103.288 66.8437) (end 103.2875 66.8432) (width 0.2) (layer "F.Cu") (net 15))
 (segment (start 103.288 69.9375) (end 103.2875 69.938) (width 0.2) (layer "F.Cu") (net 15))
 (segment (start 103.288 67.6875) (end 103.288 69.375) (width 0.2) (layer "F.Cu") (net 15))
 (segment (start 103.288 69.9375) (end 103.288 70.5) (width 0.2) (layer "F.Cu") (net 15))
 (segment (start 103.2875 69.938) (end 103.2875 70.5) (width 0.2) (layer "F.Cu") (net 15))
 (segment (start 103.288 66.8437) (end 103.288 67.6875) (width 0.2) (layer "F.Cu") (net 15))
 (segment (start 103.288 69.375) (end 103.288 67.6875) (width 0.2) (layer "F.Cu") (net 15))
 (segment (start 103.288 66) (end 103.288 66.8437) (width 0.2) (layer "F.Cu") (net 15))
 (segment (start 103.2875 66.8432) (end 103.2875 66) (width 0.2) (layer "F.Cu") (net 15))
 (segment (start 103.288 69.375) (end 103.288 69.9375) (width 0.2) (layer "F.Cu") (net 15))
 (segment (start 113.073 50.4733) (end 108.7 50.4733) (width 0.2) (layer "F.Cu") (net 5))
 (segment (start 104.77 59.941) (end 107.831 59.941) (width 0.2) (layer "F.Cu") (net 5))
 (segment (start 103.8 51.6543) (end 103.8 50.4733) (width 0.2) (layer "F.Cu") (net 5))
 (segment (start 104.156 59.3267) (end 104.77 59.941) (width 0.2) (layer "F.Cu") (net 5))
 (segment (start 118.1 55.5) (end 113.073 50.4733) (width 0.2) (layer "F.Cu") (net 5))
 (segment (start 103.8 58.9708) (end 104.156 59.3267) (width 0.2) (layer "F.Cu") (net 5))
 (segment (start 108.7 51.5) (end 108.7 50.4733) (width 0.2) (layer "F.Cu") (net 5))
 (segment (start 103.8 50.4733) (end 108.7 50.4733) (width 0.2) (layer "F.Cu") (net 5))
 (segment (start 103.8 58.045) (end 103.8 58.9708) (width 0.2) (layer "F.Cu") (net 5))
 (segment (start 104 51.8543) (end 103.8 51.6543) (width 0.2) (layer "F.Cu") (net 5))
 (segment (start 108.7 59.0717) (end 108.7 58.045) (width 0.2) (layer "F.Cu") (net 5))
 (segment (start 107.831 59.941) (end 108.7 59.0717) (width 0.2) (layer "F.Cu") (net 5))
 (via (at 104.156 59.3267) (size 0.6) (drill 0.3) (layers "F.Cu" "B.Cu") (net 5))
 (via (at 104 51.8543) (size 0.6) (drill 0.3) (layers "F.Cu" "B.Cu") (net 5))
 (segment (start 104.276 52.1303) (end 104.276 59.2066) (width 0.2) (layer "B.Cu") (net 5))
 (segment (start 104.276 59.2066) (end 104.156 59.3267) (width 0.2) (layer "B.Cu") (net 5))
 (segment (start 104 51.8543) (end 104.276 52.1303) (width 0.2) (layer "B.Cu") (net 5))
 (segment (start 110.57 57.13) (end 110.57 55.4933) (width 0.2) (layer "F.Cu") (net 12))
 (segment (start 123.373 79.325) (end 123.5 79.325) (width 0.2) (layer "F.Cu") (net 12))
 (segment (start 110.57 55.4933) (end 101.93 55.4933) (width 0.2) (layer "F.Cu") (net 12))
 (segment (start 122.684 78.6359) (end 123.373 79.325) (width 0.2) (layer "F.Cu") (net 12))
 (segment (start 101.93 55.4933) (end 101.93 57.13) (width 0.2) (layer "F.Cu") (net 12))
 (via (at 122.684 78.6359) (size 0.6) (drill 0.3) (layers "F.Cu" "B.Cu") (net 12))
 (segment (start 110.57 57.13) (end 110.57 57.6967) (width 0.2) (layer "B.Cu") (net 12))
 (segment (start 101.93 52.95) (end 101.93 57.13) (width 0.2) (layer "B.Cu") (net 12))
 (segment (start 101.93 52.95) (end 101.93 52.415) (width 0.2) (layer "B.Cu") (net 12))
 (segment (start 110.459 57.8076) (end 110.459 66.4115) (width 0.2) (layer "B.Cu") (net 12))
 (segment (start 110.57 52.95) (end 110.57 57.13) (width 0.2) (layer "B.Cu") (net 12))
 (segment (start 110.459 66.4115) (end 122.684 78.6359) (width 0.2) (layer "B.Cu") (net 12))
 (segment (start 110.57 57.6967) (end 110.459 57.8076) (width 0.2) (layer "B.Cu") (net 12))
 (segment (start 110.57 52.415) (end 110.57 52.95) (width 0.2) (layer "B.Cu") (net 12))
 (segment (start 107.5 58.045) (end 107.5 59.0717) (width 0.2) (layer "F.Cu") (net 6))
 (segment (start 109.25 78.4003) (end 110 79.15) (width 0.2) (layer "F.Cu") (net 6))
 (segment (start 107.5 59.0717) (end 105.796 59.0717) (width 0.2) (layer "F.Cu") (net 6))
 (segment (start 105 51.5) (end 105 52.7527) (width 0.2) (layer "F.Cu") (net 6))
 (segment (start 105.796 59.0717) (end 105.578 59.2898) (width 0.2) (layer "F.Cu") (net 6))
 (via (at 105 52.7527) (size 0.6) (drill 0.3) (layers "F.Cu" "B.Cu") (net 6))
 (via (at 109.25 78.4003) (size 0.6) (drill 0.3) (layers "F.Cu" "B.Cu") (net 6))
 (via (at 105.578 59.2898) (size 0.6) (drill 0.3) (layers "F.Cu" "B.Cu") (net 6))
 (segment (start 109.25 78.4003) (end 105 74.15) (width 0.2) (layer "B.Cu") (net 6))
 (segment (start 105 58.748) (end 105 52.7527) (width 0.2) (layer "B.Cu") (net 6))
 (segment (start 105 74.15) (end 105 58.748) (width 0.2) (layer "B.Cu") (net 6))
 (segment (start 105 58.748) (end 105.036 58.748) (width 0.2) (layer "B.Cu") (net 6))
 (segment (start 105.036 58.748) (end 105.578 59.2898) (width 0.2) (layer "B.Cu") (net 6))
 (segment (start 104.5 57.0183) (end 105.062 56.4566) (width 0.2) (layer "F.Cu") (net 9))
 (segment (start 116.017 78.667) (end 116.5 79.15) (width 0.2) (layer "F.Cu") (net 9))
 (segment (start 105.062 56.4566) (end 105.728 56.4566) (width 0.2) (layer "F.Cu") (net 9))
 (segment (start 108 51.5) (end 108 52.7268) (width 0.2) (layer "F.Cu") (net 9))
 (segment (start 104.5 58.045) (end 104.5 57.0183) (width 0.2) (layer "F.Cu") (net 9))
 (segment (start 111.094 78.667) (end 116.017 78.667) (width 0.2) (layer "F.Cu") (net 9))
 (via (at 108 52.7268) (size 0.6) (drill 0.3) (layers "F.Cu" "B.Cu") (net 9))
 (via (at 111.094 78.667) (size 0.6) (drill 0.3) (layers "F.Cu" "B.Cu") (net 9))
 (via (at 105.728 56.4566) (size 0.6) (drill 0.3) (layers "F.Cu" "B.Cu") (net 9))
 (segment (start 111.094 78.667) (end 108 75.5731) (width 0.2) (layer "B.Cu") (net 9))
 (segment (start 108 55.8083) (end 108 52.7268) (width 0.2) (layer "B.Cu") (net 9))
 (segment (start 108 75.5731) (end 108 55.8083) (width 0.2) (layer "B.Cu") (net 9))
 (segment (start 106.376 55.8083) (end 105.728 56.4566) (width 0.2) (layer "B.Cu") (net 9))
 (segment (start 108 55.8083) (end 106.376 55.8083) (width 0.2) (layer "B.Cu") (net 9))
 (segment (start 136.552 62.1358) (end 136.345 62.3429) (width 0.2) (layer "F.Cu") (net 13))
 (segment (start 141.325 62.5) (end 140.547 61.7216) (width 0.2) (layer "F.Cu") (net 13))
 (segment (start 136.3446 62.3429) (end 136.1375 62.55) (width 0.2) (layer "F.Cu") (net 13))
 (segment (start 136.345 62.3429) (end 136.3446 62.3429) (width 0.2) (layer "F.Cu") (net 13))
 (segment (start 136.345 62.3429) (end 136.138 62.55) (width 0.2) (layer "F.Cu") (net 13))
 (segment (start 140.547 61.7216) (end 136.966 61.7216) (width 0.2) (layer "F.Cu") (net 13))
 (segment (start 136.966 61.7216) (end 136.759 61.9287) (width 0.2) (layer "F.Cu") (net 13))
 (segment (start 136.759 61.9287) (end 136.552 62.1358) (width 0.2) (layer "F.Cu") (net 13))
 (segment (start 136.759 61.9287) (end 136.552 62.1358) (width 0.2) (layer "F.Cu") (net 13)))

